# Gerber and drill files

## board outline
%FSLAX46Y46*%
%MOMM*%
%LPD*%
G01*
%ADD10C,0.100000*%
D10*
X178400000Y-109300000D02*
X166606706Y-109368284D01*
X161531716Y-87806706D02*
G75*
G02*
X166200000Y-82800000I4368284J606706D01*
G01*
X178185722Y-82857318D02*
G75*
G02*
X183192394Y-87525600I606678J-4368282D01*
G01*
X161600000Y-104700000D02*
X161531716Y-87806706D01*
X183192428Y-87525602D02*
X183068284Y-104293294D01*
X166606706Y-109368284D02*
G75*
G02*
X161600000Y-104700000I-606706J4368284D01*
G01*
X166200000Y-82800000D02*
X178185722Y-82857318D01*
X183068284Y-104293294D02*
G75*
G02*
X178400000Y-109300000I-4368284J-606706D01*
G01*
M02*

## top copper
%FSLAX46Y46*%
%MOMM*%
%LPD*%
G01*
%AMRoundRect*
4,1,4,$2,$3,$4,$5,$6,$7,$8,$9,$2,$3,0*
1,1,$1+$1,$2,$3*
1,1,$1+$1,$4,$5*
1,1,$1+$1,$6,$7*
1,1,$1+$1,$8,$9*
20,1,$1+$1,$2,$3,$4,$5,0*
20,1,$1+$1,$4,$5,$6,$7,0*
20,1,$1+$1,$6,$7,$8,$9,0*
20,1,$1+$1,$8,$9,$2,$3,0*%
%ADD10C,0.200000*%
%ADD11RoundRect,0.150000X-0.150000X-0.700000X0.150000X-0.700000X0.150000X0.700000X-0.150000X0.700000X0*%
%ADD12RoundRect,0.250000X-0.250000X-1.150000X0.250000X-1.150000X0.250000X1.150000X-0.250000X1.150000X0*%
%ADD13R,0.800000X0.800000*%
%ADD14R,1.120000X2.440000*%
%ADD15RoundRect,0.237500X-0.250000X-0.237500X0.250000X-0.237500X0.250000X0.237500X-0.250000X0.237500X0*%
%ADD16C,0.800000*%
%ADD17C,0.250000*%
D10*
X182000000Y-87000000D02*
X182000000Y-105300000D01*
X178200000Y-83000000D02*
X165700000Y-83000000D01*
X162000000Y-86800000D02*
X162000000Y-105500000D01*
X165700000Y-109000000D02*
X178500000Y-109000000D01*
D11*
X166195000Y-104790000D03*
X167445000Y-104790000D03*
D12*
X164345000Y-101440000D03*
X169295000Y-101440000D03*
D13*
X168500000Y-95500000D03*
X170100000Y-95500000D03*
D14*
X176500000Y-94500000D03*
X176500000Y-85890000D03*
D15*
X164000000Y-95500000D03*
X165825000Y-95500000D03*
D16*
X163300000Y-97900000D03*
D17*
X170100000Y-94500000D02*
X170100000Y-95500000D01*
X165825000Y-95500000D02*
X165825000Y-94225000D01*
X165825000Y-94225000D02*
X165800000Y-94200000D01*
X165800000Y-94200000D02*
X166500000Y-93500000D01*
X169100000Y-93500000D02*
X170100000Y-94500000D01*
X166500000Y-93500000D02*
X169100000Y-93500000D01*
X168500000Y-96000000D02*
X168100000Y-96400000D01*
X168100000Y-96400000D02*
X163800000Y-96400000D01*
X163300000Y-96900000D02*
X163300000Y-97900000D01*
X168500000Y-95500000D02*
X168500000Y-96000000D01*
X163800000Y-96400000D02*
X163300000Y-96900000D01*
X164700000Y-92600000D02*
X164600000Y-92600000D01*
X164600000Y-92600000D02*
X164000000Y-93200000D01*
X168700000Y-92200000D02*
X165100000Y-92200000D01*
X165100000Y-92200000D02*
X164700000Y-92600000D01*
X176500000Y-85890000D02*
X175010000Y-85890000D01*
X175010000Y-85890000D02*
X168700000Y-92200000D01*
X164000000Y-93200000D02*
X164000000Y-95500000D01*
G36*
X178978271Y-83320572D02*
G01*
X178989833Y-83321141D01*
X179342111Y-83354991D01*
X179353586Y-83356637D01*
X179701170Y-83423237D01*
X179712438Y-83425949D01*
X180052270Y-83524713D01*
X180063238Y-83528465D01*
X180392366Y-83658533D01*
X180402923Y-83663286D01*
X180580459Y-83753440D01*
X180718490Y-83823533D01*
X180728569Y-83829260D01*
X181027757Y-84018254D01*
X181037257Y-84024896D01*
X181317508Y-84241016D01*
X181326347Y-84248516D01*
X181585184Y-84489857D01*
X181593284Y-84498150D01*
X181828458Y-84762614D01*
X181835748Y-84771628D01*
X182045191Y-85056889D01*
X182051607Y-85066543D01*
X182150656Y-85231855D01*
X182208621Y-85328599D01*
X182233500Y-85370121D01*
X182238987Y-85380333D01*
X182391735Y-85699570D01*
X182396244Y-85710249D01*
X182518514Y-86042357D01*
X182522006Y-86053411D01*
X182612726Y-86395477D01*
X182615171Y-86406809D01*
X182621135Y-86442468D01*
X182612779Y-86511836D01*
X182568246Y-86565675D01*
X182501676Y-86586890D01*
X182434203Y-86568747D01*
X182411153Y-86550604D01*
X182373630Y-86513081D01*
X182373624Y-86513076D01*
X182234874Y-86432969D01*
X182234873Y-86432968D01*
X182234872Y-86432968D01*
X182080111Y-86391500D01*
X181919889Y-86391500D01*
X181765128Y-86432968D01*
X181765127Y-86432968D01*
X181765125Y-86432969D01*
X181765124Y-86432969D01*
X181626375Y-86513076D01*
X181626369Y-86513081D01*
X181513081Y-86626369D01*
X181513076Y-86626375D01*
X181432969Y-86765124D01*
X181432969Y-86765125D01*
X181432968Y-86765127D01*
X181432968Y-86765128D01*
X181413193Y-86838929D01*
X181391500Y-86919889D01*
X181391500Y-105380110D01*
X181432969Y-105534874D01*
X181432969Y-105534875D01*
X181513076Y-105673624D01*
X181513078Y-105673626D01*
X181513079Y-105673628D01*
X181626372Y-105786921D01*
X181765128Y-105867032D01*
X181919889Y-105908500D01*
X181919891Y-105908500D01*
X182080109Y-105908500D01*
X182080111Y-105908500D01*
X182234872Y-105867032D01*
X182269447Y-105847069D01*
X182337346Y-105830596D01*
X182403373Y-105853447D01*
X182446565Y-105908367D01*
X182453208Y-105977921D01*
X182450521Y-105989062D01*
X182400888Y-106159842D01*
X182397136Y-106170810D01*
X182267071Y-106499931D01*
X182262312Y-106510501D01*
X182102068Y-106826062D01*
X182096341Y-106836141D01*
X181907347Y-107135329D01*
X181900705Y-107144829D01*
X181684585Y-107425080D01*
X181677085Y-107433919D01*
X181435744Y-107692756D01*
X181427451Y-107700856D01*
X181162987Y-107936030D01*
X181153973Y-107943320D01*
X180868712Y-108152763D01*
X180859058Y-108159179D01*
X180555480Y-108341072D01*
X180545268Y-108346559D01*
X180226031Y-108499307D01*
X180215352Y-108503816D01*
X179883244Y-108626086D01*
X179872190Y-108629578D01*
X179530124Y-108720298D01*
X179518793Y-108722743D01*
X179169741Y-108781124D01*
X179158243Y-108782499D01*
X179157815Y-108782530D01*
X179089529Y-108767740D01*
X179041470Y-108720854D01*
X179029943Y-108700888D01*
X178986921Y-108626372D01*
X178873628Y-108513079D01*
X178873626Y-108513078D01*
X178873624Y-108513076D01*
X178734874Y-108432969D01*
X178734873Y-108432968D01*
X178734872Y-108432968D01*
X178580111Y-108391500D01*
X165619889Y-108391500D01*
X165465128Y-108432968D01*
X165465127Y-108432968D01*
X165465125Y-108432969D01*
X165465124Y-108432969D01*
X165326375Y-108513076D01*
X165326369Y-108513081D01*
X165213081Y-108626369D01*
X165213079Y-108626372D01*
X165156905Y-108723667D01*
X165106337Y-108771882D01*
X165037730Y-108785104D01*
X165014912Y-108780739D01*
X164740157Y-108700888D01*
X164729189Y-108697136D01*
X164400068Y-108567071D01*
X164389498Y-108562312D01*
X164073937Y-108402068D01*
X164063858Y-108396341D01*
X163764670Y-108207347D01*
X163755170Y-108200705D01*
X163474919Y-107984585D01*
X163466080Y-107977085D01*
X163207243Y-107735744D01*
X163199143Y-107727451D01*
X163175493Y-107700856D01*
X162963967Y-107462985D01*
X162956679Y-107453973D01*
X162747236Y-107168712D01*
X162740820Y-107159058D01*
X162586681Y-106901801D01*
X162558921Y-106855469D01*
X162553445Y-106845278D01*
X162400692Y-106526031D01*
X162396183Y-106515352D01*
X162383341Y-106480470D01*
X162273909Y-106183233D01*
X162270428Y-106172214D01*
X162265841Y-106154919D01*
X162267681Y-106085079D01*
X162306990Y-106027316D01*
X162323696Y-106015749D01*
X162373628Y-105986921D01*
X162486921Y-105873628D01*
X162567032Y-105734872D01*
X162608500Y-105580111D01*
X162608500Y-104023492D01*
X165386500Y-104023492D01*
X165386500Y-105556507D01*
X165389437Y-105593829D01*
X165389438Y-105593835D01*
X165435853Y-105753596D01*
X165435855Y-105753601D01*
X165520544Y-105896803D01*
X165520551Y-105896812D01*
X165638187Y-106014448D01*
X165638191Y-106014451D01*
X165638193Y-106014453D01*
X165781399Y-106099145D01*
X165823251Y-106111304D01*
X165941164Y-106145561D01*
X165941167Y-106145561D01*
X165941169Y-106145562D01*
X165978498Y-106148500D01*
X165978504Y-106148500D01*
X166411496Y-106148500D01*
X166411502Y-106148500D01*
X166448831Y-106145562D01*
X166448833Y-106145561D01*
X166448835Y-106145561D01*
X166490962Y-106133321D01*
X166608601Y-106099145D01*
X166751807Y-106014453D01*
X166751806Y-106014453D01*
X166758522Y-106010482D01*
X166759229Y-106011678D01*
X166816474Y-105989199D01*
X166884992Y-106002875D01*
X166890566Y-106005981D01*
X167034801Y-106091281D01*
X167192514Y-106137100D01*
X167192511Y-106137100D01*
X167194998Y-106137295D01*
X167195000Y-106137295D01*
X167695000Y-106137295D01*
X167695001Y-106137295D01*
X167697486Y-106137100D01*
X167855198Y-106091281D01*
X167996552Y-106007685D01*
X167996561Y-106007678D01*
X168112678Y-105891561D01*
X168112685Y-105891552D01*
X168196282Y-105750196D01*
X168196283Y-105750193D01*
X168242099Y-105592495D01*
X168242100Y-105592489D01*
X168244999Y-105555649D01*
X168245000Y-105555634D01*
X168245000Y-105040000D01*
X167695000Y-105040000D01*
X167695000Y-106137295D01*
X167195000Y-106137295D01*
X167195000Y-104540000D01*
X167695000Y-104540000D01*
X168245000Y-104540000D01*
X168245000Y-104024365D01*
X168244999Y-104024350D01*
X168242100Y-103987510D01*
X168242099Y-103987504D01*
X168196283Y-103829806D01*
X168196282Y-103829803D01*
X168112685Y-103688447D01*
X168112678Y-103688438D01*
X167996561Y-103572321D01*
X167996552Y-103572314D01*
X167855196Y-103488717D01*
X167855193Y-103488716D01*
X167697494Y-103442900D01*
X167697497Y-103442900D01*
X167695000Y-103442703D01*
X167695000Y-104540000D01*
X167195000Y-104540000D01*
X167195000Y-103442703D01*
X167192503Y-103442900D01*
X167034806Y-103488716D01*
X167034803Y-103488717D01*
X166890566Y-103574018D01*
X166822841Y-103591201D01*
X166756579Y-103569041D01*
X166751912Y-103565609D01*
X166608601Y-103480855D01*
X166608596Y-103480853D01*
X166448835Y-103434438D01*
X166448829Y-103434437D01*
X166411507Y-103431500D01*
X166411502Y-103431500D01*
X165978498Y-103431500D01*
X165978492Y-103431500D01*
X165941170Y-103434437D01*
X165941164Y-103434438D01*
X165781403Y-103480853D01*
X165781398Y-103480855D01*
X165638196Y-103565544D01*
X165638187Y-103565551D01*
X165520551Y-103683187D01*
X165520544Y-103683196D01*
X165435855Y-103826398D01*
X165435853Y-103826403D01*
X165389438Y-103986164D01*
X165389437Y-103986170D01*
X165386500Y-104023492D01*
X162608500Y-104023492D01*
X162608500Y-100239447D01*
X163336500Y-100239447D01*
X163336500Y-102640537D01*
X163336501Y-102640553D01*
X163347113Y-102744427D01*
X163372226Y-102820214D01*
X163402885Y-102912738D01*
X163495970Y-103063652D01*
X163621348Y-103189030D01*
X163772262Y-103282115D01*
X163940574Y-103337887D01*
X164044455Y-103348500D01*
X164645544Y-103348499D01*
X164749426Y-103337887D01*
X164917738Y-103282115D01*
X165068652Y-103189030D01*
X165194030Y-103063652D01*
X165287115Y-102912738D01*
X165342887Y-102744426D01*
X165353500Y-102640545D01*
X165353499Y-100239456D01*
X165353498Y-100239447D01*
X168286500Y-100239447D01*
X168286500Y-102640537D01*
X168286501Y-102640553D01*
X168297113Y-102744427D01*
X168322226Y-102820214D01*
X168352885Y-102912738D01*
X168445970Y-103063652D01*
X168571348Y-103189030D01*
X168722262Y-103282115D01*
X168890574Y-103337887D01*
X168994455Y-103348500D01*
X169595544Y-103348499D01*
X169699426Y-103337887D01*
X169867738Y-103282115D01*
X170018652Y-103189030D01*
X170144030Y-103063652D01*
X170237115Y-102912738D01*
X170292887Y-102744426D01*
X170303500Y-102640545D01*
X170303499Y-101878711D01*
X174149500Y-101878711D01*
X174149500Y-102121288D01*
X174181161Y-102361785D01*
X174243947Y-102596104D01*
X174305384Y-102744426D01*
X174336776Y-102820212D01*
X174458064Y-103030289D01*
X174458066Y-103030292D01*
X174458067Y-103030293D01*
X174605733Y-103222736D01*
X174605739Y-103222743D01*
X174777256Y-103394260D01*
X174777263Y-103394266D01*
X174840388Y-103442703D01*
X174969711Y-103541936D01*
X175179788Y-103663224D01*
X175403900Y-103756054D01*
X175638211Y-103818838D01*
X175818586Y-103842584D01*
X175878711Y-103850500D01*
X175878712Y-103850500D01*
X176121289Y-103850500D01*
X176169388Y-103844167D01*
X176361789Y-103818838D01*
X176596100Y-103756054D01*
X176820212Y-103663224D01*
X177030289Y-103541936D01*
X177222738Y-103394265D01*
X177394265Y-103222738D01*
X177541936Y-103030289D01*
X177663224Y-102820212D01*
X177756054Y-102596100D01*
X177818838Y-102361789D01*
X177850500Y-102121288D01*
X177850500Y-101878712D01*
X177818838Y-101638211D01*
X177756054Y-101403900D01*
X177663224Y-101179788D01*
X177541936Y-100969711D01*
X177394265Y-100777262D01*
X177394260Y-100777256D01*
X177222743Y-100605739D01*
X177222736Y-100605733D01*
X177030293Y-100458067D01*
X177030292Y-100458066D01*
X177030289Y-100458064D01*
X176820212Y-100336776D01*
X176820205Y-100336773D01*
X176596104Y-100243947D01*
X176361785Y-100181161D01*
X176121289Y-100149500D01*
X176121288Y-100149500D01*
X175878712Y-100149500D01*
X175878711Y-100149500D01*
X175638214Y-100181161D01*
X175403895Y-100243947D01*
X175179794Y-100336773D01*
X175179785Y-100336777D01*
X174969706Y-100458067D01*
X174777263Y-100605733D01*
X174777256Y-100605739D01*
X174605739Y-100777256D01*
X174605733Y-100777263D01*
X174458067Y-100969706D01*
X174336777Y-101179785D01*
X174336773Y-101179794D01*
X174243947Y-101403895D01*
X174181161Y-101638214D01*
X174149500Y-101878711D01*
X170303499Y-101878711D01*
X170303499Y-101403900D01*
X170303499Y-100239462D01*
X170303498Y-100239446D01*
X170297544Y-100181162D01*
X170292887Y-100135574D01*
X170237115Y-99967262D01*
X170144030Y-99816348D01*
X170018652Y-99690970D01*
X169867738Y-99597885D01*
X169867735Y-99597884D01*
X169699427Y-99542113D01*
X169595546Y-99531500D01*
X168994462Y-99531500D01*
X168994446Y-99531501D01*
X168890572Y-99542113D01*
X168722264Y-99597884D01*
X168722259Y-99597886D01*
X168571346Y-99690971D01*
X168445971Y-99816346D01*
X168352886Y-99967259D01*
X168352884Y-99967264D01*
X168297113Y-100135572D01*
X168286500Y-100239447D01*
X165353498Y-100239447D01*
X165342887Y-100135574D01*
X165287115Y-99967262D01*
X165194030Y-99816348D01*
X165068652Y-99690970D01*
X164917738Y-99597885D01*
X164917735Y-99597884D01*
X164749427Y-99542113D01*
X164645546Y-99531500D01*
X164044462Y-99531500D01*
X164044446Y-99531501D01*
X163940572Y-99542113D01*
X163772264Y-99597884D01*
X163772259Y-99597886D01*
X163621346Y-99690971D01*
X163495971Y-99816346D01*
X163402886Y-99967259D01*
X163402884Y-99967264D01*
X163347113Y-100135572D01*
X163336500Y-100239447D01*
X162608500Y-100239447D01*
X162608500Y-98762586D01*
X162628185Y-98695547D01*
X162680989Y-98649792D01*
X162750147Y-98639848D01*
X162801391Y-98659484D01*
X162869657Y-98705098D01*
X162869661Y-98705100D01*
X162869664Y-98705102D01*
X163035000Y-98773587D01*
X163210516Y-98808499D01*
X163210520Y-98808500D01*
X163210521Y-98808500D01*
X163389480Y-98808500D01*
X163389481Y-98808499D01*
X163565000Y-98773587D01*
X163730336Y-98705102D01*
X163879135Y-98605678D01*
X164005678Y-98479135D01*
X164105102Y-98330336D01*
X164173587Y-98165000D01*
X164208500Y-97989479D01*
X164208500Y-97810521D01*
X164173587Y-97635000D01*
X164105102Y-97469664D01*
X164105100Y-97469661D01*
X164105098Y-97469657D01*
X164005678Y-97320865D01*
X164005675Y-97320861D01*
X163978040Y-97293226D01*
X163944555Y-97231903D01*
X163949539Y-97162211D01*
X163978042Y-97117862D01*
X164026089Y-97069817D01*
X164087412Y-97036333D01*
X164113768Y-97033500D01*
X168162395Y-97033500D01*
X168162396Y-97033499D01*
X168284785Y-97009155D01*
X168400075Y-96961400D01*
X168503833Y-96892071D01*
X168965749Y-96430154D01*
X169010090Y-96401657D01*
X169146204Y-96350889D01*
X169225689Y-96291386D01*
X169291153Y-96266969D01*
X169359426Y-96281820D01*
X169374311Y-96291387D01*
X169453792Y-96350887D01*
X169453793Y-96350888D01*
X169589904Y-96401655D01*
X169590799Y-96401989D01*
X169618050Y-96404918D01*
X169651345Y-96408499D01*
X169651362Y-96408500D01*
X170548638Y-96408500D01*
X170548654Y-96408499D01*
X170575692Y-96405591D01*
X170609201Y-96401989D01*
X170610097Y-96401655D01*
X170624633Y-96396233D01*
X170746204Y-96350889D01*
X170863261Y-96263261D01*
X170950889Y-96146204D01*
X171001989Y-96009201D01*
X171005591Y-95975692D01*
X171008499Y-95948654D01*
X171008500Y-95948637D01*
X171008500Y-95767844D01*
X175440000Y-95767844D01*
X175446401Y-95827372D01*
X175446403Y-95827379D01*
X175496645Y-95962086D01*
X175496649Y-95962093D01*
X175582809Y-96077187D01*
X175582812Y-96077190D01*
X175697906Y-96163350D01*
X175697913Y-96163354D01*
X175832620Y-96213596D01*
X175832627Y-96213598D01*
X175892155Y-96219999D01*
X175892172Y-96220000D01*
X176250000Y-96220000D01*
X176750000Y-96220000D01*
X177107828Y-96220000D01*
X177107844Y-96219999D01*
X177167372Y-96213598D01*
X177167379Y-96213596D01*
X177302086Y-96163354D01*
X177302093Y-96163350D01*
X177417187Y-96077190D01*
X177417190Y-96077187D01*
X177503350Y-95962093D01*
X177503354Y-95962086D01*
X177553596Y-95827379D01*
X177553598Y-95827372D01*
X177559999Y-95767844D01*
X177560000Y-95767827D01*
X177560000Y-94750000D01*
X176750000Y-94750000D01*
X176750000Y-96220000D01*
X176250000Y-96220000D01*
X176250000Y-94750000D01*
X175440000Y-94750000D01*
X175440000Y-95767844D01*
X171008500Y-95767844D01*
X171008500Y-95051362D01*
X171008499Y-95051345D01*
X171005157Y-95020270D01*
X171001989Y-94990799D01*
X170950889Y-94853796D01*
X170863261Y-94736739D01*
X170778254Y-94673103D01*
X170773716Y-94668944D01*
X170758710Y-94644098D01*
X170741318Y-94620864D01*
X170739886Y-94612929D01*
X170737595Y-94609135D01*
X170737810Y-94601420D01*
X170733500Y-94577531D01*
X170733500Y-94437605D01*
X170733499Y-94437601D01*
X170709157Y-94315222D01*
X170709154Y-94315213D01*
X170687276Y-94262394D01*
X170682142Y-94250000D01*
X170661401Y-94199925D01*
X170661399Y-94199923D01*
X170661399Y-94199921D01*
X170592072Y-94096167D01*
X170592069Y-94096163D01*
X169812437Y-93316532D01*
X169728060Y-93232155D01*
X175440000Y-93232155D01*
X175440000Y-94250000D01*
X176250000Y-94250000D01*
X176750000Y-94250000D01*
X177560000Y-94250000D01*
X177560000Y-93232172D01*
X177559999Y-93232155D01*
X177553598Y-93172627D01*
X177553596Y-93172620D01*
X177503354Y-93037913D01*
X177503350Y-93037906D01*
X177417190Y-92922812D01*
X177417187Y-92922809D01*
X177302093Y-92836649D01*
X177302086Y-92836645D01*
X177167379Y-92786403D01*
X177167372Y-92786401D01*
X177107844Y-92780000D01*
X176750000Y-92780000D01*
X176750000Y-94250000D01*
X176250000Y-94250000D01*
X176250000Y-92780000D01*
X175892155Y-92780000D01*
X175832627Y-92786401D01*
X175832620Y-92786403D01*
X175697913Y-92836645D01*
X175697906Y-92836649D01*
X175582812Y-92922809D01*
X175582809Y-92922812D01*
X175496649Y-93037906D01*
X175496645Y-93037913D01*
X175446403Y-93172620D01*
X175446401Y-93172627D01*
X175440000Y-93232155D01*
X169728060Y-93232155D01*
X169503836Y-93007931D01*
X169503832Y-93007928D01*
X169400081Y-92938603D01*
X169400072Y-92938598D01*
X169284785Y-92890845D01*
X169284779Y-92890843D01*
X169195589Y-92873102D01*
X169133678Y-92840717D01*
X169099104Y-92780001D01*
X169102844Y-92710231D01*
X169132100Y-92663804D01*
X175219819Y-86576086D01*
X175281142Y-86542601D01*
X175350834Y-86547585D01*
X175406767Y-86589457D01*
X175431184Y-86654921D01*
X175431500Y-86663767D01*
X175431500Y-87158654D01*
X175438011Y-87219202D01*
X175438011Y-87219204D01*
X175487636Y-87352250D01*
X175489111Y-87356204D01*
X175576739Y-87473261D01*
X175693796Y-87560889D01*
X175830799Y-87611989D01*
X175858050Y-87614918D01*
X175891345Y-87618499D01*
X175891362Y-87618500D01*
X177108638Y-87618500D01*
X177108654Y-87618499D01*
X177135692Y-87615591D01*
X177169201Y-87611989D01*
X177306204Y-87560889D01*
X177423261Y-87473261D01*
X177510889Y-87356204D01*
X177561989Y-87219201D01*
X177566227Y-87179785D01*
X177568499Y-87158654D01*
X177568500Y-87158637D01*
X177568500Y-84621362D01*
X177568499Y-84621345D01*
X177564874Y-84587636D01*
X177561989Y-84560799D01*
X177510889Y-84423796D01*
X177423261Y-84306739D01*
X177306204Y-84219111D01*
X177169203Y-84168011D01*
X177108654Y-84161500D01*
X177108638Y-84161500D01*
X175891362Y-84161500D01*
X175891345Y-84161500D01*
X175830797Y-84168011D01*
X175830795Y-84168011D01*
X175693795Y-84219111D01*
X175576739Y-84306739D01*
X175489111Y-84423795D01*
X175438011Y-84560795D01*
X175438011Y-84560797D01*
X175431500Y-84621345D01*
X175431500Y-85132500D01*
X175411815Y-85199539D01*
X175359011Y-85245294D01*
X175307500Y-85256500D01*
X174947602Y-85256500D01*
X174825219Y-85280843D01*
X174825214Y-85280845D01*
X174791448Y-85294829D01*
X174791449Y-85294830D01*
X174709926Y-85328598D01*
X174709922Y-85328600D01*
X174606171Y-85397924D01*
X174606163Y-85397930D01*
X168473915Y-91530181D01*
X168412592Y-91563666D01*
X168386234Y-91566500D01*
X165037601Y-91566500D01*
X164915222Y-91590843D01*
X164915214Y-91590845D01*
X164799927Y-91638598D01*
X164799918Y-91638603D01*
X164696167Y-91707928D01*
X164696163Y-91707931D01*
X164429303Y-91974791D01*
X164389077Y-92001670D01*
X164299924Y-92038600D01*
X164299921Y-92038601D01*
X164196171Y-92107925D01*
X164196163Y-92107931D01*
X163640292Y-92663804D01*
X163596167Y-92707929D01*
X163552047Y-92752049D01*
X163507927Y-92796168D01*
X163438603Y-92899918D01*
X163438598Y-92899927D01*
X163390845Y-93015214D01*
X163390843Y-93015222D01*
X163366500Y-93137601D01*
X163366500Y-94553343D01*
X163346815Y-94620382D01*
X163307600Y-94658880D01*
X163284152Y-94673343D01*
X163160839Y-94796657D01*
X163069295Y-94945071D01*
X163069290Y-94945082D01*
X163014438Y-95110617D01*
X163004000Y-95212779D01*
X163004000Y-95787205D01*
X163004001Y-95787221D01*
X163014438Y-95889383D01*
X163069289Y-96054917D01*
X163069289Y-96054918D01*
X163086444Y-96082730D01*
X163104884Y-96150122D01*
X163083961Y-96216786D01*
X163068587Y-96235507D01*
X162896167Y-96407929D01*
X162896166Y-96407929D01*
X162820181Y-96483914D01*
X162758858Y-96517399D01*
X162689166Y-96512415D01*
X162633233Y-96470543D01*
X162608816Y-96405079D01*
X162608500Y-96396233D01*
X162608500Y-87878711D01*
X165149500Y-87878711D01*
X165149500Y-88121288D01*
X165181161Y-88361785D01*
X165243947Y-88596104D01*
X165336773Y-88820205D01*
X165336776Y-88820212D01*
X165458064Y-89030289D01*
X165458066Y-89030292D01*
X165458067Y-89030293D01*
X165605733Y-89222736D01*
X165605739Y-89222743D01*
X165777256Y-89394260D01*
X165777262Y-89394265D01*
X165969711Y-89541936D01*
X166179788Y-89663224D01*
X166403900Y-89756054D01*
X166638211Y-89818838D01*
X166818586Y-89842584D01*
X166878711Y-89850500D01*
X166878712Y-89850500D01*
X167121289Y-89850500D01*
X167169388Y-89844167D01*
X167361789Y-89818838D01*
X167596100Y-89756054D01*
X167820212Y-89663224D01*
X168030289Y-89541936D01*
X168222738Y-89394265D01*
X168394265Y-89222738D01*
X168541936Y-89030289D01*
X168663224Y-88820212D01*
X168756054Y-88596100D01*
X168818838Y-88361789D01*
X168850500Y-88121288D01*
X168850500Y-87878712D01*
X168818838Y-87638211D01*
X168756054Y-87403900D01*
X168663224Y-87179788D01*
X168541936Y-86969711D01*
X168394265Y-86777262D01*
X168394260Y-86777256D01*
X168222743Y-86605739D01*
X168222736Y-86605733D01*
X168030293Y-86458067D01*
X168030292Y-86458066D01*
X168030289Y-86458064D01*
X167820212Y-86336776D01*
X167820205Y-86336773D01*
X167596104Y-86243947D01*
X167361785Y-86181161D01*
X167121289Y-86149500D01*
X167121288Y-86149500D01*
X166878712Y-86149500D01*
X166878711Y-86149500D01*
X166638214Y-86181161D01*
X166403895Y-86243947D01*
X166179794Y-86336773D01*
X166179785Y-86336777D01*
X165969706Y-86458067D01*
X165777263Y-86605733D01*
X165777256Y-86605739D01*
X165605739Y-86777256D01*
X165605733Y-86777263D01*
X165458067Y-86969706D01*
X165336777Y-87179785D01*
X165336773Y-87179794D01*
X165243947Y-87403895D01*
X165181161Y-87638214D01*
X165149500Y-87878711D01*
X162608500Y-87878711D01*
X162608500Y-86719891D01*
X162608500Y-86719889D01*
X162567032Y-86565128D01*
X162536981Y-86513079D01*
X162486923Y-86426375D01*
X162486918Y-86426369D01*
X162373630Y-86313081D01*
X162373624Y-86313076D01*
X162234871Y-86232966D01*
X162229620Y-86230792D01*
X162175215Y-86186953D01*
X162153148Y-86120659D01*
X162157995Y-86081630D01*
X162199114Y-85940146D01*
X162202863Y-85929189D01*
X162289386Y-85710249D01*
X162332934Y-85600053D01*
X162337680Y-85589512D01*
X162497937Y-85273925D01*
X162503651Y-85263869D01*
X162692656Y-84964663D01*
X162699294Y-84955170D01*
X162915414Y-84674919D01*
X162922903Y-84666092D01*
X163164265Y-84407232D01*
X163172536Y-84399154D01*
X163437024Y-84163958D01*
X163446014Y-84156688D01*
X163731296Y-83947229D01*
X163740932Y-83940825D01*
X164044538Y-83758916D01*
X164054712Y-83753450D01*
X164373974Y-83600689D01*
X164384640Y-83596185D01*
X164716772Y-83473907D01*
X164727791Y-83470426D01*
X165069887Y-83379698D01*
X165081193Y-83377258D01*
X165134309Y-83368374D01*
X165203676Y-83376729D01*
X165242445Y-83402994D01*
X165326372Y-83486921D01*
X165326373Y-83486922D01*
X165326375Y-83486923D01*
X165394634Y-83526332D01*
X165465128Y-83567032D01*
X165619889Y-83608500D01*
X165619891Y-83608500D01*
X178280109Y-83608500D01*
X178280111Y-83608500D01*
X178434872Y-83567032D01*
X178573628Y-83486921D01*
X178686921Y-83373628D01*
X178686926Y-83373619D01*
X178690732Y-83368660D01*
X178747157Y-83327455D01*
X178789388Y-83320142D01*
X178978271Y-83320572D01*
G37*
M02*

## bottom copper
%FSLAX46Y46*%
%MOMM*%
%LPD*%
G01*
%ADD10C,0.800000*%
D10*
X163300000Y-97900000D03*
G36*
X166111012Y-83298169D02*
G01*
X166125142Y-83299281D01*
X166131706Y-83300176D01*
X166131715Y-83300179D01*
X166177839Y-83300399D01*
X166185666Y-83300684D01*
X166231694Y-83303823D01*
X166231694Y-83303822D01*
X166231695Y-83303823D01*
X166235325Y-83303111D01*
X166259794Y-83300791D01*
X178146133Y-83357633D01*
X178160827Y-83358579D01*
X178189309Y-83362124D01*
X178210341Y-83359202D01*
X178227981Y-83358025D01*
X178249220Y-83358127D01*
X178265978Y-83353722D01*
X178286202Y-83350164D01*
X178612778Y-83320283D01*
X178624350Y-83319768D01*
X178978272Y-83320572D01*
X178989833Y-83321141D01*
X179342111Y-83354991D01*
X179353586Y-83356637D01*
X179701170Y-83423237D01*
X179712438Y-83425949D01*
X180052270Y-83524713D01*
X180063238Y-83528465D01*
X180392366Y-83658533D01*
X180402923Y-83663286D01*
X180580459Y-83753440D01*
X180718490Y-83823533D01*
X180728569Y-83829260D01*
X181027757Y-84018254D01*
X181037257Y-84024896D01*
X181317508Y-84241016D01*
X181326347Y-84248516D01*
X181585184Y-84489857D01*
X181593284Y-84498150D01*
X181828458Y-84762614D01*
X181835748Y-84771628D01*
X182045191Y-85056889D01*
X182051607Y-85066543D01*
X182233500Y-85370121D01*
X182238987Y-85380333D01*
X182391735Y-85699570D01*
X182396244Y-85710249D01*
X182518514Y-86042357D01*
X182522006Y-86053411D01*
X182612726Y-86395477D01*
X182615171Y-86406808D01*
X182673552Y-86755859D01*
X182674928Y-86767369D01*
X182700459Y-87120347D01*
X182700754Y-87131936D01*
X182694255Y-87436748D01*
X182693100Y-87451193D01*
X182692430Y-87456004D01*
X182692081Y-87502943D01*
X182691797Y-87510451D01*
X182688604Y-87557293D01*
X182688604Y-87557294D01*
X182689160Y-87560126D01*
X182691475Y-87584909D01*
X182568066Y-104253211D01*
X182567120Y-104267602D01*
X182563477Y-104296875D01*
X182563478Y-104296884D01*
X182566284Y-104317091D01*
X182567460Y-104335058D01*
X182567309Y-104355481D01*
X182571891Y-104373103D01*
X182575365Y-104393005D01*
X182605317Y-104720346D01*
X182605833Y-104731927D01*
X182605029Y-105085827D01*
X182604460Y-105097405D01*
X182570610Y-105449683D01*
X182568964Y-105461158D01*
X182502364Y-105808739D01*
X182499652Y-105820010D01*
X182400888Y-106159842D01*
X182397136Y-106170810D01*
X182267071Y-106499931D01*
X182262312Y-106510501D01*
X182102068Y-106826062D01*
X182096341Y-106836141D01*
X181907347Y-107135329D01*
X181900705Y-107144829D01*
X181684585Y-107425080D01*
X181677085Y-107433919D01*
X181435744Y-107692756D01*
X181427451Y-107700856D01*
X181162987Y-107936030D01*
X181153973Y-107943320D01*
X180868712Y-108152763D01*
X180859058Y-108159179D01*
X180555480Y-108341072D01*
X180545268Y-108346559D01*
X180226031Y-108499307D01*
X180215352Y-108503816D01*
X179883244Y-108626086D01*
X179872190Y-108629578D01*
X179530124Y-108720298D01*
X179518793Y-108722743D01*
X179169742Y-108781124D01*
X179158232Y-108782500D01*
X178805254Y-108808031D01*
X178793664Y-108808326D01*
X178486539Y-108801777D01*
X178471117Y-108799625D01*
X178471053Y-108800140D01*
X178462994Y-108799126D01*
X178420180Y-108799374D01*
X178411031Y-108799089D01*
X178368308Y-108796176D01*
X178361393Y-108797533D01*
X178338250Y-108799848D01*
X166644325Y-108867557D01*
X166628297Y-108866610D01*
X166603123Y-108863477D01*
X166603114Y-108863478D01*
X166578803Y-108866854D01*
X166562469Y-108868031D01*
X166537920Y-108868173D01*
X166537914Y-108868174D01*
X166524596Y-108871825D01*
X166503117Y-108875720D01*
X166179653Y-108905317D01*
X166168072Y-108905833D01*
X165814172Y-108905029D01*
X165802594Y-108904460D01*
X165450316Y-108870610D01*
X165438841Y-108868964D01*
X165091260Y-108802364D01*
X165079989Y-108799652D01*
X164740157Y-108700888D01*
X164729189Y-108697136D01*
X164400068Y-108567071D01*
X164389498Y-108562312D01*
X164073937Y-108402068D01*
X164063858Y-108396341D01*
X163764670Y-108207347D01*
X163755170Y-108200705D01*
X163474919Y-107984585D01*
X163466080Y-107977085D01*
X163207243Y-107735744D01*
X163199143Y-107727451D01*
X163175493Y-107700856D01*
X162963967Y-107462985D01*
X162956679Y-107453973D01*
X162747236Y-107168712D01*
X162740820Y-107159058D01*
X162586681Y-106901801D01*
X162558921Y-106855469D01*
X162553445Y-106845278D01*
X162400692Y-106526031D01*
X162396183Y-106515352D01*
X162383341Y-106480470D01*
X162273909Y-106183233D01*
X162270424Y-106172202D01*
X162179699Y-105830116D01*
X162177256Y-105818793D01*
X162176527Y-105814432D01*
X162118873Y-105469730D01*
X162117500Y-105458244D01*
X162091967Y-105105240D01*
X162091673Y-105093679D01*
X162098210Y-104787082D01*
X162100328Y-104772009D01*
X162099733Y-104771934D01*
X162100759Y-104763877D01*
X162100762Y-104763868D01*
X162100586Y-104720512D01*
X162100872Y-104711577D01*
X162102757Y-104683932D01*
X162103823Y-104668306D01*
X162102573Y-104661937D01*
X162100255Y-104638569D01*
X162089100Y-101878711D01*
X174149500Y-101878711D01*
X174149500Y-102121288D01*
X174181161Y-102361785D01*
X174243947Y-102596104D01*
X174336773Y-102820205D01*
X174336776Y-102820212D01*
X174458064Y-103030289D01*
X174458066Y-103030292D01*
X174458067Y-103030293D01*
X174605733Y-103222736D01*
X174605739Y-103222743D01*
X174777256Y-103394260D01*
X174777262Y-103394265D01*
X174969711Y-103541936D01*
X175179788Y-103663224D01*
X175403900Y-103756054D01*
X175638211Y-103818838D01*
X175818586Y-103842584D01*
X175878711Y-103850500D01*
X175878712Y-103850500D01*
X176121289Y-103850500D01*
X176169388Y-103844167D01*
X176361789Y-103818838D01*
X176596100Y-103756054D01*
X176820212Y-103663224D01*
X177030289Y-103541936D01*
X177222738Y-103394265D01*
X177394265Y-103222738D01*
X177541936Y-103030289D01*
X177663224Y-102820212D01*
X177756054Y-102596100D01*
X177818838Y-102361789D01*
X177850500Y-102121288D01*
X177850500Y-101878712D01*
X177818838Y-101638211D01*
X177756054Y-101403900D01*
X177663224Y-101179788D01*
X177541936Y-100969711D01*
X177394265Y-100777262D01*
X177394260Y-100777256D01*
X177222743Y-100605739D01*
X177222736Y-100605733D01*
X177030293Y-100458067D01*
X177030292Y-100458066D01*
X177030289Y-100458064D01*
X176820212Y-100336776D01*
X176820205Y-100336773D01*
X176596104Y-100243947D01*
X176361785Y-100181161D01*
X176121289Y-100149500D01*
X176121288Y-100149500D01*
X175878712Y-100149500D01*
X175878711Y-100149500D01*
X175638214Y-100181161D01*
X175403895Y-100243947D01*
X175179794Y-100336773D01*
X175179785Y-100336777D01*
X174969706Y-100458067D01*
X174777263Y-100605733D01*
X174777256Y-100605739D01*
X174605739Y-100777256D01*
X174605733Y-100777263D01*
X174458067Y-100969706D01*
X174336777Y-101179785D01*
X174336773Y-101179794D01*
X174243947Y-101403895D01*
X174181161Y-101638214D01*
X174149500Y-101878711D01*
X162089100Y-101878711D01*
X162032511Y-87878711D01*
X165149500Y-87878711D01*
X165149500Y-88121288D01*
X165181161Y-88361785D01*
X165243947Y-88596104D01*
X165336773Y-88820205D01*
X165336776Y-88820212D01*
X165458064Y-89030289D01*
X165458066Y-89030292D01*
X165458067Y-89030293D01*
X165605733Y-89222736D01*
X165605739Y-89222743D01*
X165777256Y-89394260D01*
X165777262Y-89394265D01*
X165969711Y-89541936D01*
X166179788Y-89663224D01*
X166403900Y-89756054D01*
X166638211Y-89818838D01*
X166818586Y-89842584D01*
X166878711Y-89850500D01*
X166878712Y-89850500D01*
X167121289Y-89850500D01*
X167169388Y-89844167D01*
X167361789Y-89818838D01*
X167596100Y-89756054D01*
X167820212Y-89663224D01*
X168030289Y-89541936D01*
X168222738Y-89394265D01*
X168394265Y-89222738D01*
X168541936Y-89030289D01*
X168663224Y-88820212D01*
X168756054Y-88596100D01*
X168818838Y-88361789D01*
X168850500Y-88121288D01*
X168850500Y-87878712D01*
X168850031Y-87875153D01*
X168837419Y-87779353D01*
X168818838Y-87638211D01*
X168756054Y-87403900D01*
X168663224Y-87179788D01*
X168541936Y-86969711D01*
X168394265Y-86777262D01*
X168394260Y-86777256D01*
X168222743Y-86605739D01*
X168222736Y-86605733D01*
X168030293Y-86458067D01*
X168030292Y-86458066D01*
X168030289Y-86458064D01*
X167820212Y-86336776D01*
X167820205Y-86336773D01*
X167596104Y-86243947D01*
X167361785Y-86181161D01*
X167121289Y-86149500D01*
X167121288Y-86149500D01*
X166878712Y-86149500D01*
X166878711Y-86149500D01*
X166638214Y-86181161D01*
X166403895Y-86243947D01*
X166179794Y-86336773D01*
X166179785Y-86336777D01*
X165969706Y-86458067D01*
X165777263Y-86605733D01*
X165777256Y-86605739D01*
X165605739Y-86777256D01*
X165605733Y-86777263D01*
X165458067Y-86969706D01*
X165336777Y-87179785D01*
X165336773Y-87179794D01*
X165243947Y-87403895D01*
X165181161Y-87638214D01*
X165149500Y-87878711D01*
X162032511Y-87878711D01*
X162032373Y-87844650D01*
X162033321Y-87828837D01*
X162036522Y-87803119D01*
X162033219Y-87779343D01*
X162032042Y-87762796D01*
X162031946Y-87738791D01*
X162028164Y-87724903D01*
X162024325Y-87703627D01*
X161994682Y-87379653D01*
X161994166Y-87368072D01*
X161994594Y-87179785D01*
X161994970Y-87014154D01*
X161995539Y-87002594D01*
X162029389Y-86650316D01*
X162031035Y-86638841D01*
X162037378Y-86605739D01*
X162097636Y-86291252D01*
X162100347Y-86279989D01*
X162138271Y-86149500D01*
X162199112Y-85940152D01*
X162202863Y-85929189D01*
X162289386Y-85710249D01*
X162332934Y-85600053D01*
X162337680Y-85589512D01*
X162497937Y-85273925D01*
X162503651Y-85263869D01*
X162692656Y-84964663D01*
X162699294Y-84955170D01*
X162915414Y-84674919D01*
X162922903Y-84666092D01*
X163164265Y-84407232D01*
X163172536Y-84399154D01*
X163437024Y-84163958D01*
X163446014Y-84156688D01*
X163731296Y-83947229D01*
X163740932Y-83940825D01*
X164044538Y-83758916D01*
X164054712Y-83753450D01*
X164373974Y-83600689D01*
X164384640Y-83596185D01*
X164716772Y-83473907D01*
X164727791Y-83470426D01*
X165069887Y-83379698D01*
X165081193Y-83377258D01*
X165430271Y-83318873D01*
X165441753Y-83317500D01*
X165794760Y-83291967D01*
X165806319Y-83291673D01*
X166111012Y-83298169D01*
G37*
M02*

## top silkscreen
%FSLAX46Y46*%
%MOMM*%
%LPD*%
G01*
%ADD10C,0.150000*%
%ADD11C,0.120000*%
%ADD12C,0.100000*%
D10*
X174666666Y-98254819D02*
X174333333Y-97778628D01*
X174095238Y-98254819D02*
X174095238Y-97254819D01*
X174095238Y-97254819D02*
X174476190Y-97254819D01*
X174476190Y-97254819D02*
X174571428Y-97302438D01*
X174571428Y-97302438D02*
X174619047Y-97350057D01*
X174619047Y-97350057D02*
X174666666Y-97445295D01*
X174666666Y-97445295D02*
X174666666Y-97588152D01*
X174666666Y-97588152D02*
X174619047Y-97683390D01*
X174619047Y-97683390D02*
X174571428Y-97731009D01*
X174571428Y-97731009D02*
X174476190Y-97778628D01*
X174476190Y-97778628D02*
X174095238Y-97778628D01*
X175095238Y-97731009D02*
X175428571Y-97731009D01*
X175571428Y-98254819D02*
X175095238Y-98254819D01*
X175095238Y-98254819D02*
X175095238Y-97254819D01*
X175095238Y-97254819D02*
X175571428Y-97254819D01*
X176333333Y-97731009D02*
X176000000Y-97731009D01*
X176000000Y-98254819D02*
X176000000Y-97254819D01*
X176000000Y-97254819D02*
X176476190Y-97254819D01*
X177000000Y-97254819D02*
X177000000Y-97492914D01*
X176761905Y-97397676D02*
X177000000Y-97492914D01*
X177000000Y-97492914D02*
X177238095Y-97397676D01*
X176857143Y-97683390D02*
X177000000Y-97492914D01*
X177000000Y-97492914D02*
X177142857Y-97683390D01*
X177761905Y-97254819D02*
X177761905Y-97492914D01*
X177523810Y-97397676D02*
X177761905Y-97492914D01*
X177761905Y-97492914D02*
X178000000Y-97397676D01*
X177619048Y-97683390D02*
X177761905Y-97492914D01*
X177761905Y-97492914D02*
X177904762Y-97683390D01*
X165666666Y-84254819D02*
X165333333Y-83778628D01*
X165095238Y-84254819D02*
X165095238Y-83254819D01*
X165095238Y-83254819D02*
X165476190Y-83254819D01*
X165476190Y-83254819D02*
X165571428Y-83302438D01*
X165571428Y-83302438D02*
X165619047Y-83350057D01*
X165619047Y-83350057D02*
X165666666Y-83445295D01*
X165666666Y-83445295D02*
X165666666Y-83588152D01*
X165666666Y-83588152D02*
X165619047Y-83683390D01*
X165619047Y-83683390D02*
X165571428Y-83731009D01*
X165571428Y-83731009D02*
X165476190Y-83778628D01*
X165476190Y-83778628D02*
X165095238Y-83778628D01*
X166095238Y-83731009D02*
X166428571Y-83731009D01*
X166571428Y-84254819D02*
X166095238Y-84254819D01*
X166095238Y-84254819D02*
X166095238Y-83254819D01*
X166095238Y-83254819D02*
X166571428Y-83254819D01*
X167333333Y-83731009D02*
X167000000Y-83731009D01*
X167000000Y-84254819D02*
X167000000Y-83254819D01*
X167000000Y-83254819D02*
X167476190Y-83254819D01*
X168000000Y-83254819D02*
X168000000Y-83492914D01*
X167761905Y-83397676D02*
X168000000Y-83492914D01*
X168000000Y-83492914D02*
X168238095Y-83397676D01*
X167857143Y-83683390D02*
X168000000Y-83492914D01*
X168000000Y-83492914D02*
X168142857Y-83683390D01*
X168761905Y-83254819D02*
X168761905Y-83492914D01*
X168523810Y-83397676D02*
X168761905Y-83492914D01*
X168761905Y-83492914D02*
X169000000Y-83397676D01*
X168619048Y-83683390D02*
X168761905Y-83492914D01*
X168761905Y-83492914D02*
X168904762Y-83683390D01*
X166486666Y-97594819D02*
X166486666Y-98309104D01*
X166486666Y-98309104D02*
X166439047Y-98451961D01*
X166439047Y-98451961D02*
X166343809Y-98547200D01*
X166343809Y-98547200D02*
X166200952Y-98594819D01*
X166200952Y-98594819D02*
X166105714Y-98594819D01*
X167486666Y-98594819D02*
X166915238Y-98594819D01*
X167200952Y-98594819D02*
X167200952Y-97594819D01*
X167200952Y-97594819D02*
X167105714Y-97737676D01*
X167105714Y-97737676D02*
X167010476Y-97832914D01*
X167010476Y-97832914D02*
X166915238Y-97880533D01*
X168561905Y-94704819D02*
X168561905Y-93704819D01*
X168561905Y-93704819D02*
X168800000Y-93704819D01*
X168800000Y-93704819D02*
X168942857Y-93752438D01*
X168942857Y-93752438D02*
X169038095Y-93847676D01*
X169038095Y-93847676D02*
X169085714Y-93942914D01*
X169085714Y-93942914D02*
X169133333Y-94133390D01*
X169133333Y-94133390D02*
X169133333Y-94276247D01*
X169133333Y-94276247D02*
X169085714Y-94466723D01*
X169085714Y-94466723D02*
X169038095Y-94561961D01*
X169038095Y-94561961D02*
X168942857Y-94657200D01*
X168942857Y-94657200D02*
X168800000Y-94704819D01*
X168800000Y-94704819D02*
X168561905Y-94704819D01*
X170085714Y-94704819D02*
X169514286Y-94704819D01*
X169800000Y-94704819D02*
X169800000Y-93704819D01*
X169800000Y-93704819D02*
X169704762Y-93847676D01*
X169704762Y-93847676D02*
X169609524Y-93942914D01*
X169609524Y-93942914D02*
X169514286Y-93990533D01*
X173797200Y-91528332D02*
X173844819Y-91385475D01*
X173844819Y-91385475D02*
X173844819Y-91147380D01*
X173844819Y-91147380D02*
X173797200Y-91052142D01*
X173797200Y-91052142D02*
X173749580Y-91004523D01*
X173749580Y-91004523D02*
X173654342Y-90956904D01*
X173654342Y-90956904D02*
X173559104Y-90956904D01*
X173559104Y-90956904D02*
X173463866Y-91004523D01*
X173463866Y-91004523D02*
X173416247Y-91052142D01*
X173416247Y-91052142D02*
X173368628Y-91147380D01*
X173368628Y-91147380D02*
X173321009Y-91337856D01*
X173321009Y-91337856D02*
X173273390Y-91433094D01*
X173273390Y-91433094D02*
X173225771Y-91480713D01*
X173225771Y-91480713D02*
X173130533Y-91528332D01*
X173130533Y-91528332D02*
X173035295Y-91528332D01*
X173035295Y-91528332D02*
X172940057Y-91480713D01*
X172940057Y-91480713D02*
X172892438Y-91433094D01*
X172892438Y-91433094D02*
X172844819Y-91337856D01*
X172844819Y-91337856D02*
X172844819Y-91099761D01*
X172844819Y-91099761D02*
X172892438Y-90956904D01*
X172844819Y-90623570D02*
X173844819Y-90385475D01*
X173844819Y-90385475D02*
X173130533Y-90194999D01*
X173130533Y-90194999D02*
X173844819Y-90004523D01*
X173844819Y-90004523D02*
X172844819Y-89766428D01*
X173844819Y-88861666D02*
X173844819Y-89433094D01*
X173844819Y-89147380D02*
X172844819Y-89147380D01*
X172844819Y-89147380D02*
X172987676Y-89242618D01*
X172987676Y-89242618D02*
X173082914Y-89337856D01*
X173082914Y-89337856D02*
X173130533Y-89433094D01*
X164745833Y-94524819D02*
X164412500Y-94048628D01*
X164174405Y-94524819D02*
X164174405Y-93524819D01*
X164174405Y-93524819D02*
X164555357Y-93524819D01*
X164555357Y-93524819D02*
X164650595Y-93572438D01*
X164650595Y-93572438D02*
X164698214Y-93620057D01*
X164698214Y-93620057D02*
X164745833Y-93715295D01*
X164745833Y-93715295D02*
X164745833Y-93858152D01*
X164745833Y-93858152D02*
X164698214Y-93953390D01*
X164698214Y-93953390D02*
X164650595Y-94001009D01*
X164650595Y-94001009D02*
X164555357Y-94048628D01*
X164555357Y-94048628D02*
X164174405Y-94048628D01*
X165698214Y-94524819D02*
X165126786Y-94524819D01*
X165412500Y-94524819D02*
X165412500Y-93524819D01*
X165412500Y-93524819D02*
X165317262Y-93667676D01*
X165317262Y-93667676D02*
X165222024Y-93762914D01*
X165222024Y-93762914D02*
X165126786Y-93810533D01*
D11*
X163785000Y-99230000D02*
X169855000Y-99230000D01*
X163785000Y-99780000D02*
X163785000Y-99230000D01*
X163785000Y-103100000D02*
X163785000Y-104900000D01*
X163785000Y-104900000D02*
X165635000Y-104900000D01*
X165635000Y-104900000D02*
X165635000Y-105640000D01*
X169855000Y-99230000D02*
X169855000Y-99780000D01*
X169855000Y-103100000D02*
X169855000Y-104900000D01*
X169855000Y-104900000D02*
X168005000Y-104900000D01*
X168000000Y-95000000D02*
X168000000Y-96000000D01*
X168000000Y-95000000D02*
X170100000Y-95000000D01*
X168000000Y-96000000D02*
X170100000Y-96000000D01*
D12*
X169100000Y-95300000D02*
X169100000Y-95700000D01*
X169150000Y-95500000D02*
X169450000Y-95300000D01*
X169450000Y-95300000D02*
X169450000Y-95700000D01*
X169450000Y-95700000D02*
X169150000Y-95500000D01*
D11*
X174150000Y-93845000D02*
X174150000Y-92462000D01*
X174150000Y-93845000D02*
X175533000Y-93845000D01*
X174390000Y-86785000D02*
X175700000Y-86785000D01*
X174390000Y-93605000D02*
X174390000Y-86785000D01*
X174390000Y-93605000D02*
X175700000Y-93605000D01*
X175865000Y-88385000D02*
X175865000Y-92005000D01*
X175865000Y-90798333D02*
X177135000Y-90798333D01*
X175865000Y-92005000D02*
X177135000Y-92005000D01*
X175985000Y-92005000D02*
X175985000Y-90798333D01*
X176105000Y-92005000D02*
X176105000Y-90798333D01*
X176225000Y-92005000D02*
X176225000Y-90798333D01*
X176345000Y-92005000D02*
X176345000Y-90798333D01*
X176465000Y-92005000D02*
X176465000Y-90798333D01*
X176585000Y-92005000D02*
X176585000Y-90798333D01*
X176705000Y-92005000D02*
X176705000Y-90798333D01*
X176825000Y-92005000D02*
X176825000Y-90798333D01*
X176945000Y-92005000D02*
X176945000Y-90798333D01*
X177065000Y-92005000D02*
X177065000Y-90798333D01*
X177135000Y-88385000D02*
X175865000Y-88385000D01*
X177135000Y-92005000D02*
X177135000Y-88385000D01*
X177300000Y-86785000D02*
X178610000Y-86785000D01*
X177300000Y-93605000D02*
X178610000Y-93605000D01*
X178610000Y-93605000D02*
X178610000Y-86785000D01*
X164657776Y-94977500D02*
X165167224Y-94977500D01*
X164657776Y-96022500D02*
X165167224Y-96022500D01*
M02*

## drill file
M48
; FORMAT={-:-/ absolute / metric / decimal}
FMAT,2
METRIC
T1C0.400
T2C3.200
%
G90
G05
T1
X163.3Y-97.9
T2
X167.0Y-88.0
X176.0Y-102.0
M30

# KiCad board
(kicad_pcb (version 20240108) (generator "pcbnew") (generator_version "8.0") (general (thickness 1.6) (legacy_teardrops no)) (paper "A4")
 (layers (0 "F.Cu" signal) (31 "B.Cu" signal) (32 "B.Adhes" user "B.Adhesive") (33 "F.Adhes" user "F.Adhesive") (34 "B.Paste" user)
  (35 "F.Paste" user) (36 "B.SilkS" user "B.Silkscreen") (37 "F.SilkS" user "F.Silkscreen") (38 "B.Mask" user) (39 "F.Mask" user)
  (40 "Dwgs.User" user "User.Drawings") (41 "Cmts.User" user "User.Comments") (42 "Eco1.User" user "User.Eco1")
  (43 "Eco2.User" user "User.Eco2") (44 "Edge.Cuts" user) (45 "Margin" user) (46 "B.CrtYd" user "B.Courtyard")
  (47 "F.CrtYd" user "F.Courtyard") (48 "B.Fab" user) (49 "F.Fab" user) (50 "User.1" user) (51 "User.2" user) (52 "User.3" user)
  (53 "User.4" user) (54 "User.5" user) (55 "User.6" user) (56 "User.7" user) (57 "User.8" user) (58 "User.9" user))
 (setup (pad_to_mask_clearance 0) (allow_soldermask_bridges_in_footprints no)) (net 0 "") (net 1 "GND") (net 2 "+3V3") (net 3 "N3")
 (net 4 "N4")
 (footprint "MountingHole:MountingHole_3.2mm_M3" (layer "F.Cu") (at 176 102)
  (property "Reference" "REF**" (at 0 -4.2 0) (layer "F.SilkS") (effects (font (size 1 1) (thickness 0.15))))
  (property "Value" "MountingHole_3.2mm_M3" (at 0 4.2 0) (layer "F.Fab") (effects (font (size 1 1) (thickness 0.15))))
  (pad "" np_thru_hole circle (at 0 0) (size 3.2 3.2) (drill 3.2) (layers "*.Cu" "*.Mask")))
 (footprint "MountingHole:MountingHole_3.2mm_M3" (layer "F.Cu") (at 167 88)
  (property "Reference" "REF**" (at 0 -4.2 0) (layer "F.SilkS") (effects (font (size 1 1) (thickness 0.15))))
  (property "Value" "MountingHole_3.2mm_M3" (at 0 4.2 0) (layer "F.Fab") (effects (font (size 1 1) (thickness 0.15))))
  (pad "" np_thru_hole circle (at 0 0) (size 3.2 3.2) (drill 3.2) (layers "*.Cu" "*.Mask")))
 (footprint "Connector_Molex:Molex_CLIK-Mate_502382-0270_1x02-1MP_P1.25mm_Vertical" (layer "F.Cu") (at 166.82 102.84)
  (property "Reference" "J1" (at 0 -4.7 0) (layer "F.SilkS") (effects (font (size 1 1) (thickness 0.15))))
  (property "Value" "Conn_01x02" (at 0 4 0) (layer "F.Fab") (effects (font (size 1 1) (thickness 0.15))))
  (fp_line (start -3.035 -3.61) (end 3.035 -3.61) (stroke (width 0.12) (type solid)) (layer "F.SilkS"))
  (fp_line (start -3.035 -3.06) (end -3.035 -3.61) (stroke (width 0.12) (type solid)) (layer "F.SilkS"))
  (fp_line (start -3.035 0.26) (end -3.035 2.06) (stroke (width 0.12) (type solid)) (layer "F.SilkS"))
  (fp_line (start -3.035 2.06) (end -1.185 2.06) (stroke (width 0.12) (type solid)) (layer "F.SilkS"))
  (fp_line (start -1.185 2.06) (end -1.185 2.8) (stroke (width 0.12) (type solid)) (layer "F.SilkS"))
  (fp_line (start 3.035 -3.61) (end 3.035 -3.06) (stroke (width 0.12) (type solid)) (layer "F.SilkS"))
  (fp_line (start 3.035 0.26) (end 3.035 2.06) (stroke (width 0.12) (type solid)) (layer "F.SilkS"))
  (fp_line (start 3.035 2.06) (end 1.185 2.06) (stroke (width 0.12) (type solid)) (layer "F.SilkS"))
  (pad "1" smd roundrect (at -0.625 1.95) (size 0.6 1.7) (layers "F.Cu" "F.Paste" "F.Mask") (roundrect_rratio 0.25) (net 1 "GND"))
  (pad "2" smd roundrect (at 0.625 1.95) (size 0.6 1.7) (layers "F.Cu" "F.Paste" "F.Mask") (roundrect_rratio 0.25) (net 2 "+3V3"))
  (pad "MP" smd roundrect (at -2.475 -1.4) (size 1 2.8) (layers "F.Cu" "F.Paste" "F.Mask") (roundrect_rratio 0.25))
  (pad "MP" smd roundrect (at 2.475 -1.4) (size 1 2.8) (layers "F.Cu" "F.Paste" "F.Mask") (roundrect_rratio 0.25)))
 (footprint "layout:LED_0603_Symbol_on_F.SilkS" (layer "F.Cu") (at 169.3 95.5)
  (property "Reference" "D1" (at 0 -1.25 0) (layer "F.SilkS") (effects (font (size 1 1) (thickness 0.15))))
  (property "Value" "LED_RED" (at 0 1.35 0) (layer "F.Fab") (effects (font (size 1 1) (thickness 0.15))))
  (fp_line (start -1.3 -0.5) (end -1.3 0.5) (stroke (width 0.12) (type solid)) (layer "F.SilkS"))
  (fp_line (start -1.3 -0.5) (end 0.8 -0.5) (stroke (width 0.12) (type solid)) (layer "F.SilkS"))
  (fp_line (start -1.3 0.5) (end 0.8 0.5) (stroke (width 0.12) (type solid)) (layer "F.SilkS"))
  (fp_line (start -0.2 -0.2) (end -0.2 0.2) (stroke (width 0.1) (type solid)) (layer "F.SilkS"))
  (fp_line (start -0.15 0) (end 0.15 -0.2) (stroke (width 0.1) (type solid)) (layer "F.SilkS"))
  (fp_line (start 0.15 -0.2) (end 0.15 0.2) (stroke (width 0.1) (type solid)) (layer "F.SilkS"))
  (fp_line (start 0.15 0.2) (end -0.15 0) (stroke (width 0.1) (type solid)) (layer "F.SilkS"))
  (pad "1" smd rect (at -0.8 0 180) (size 0.8 0.8) (layers "F.Cu" "F.Paste" "F.Mask") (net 1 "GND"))
  (pad "2" smd rect (at 0.8 0 180) (size 0.8 0.8) (layers "F.Cu" "F.Paste" "F.Mask") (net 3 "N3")))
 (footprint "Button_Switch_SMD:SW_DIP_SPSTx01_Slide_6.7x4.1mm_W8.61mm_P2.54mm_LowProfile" (layer "F.Cu") (at 176.5 90.195 90)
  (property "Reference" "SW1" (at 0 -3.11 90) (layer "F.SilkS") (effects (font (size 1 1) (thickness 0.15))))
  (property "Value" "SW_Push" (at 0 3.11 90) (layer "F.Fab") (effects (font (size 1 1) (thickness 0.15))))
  (fp_line (start -3.65 -2.35) (end -2.267 -2.35) (stroke (width 0.12) (type solid)) (layer "F.SilkS"))
  (fp_line (start -3.65 -2.35) (end -3.65 -0.967) (stroke (width 0.12) (type solid)) (layer "F.SilkS"))
  (fp_line (start 3.41 -2.11) (end 3.41 -0.8) (stroke (width 0.12) (type solid)) (layer "F.SilkS"))
  (fp_line (start -3.41 -2.11) (end 3.41 -2.11) (stroke (width 0.12) (type solid)) (layer "F.SilkS"))
  (fp_line (start -3.41 -2.11) (end -3.41 -0.8) (stroke (width 0.12) (type solid)) (layer "F.SilkS"))
  (fp_line (start 1.81 -0.635) (end -1.81 -0.635) (stroke (width 0.12) (type solid)) (layer "F.SilkS"))
  (fp_line (start -0.603333 -0.635) (end -0.603333 0.635) (stroke (width 0.12) (type solid)) (layer "F.SilkS"))
  (fp_line (start -1.81 -0.635) (end -1.81 0.635) (stroke (width 0.12) (type solid)) (layer "F.SilkS"))
  (fp_line (start -1.81 -0.515) (end -0.603333 -0.515) (stroke (width 0.12) (type solid)) (layer "F.SilkS"))
  (fp_line (start -1.81 -0.395) (end -0.603333 -0.395) (stroke (width 0.12) (type solid)) (layer "F.SilkS"))
  (fp_line (start -1.81 -0.275) (end -0.603333 -0.275) (stroke (width 0.12) (type solid)) (layer "F.SilkS"))
  (fp_line (start -1.81 -0.155) (end -0.603333 -0.155) (stroke (width 0.12) (type solid)) (layer "F.SilkS"))
  (fp_line (start -1.81 -0.035) (end -0.603333 -0.035) (stroke (width 0.12) (type solid)) (layer "F.SilkS"))
  (fp_line (start -1.81 0.085) (end -0.603333 0.085) (stroke (width 0.12) (type solid)) (layer "F.SilkS"))
  (fp_line (start -1.81 0.205) (end -0.603333 0.205) (stroke (width 0.12) (type solid)) (layer "F.SilkS"))
  (fp_line (start -1.81 0.325) (end -0.603333 0.325) (stroke (width 0.12) (type solid)) (layer "F.SilkS"))
  (fp_line (start -1.81 0.445) (end -0.603333 0.445) (stroke (width 0.12) (type solid)) (layer "F.SilkS"))
  (fp_line (start -1.81 0.565) (end -0.603333 0.565) (stroke (width 0.12) (type solid)) (layer "F.SilkS"))
  (fp_line (start 1.81 0.635) (end 1.81 -0.635) (stroke (width 0.12) (type solid)) (layer "F.SilkS"))
  (fp_line (start -1.81 0.635) (end 1.81 0.635) (stroke (width 0.12) (type solid)) (layer "F.SilkS"))
  (fp_line (start 3.41 0.8) (end 3.41 2.11) (stroke (width 0.12) (type solid)) (layer "F.SilkS"))
  (fp_line (start -3.41 0.8) (end -3.41 2.11) (stroke (width 0.12) (type solid)) (layer "F.SilkS"))
  (fp_line (start -3.41 2.11) (end 3.41 2.11) (stroke (width 0.12) (type solid)) (layer "F.SilkS"))
  (pad "1" smd rect (at -4.305 0 90) (size 2.44 1.12) (layers "F.Cu" "F.Paste" "F.Mask") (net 2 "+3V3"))
  (pad "2" smd rect (at 4.305 0 90) (size 2.44 1.12) (layers "F.Cu" "F.Paste" "F.Mask") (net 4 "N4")))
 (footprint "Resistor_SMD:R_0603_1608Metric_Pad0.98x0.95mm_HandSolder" (layer "F.Cu") (at 164.9125 95.5)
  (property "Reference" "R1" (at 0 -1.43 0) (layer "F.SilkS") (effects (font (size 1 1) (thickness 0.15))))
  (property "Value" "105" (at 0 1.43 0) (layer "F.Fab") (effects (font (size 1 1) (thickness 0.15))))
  (fp_line (start -0.254724 -0.5225) (end 0.254724 -0.5225) (stroke (width 0.12) (type solid)) (layer "F.SilkS"))
  (fp_line (start -0.254724 0.5225) (end 0.254724 0.5225) (stroke (width 0.12) (type solid)) (layer "F.SilkS"))
  (pad "1" smd roundrect (at -0.9125 0) (size 0.975 0.95) (layers "F.Cu" "F.Paste" "F.Mask") (roundrect_rratio 0.25) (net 4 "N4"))
  (pad "2" smd roundrect (at 0.9125 0) (size 0.975 0.95) (layers "F.Cu" "F.Paste" "F.Mask") (roundrect_rratio 0.25) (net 3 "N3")))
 (gr_line (start 182 87) (end 182 105.3) (stroke (width 0.2) (type default)) (layer "F.Cu"))
 (gr_line (start 178.2 83) (end 165.7 83) (stroke (width 0.2) (type default)) (layer "F.Cu"))
 (gr_line (start 162 86.8) (end 162 105.5) (stroke (width 0.2) (type default)) (layer "F.Cu"))
 (gr_line (start 165.7 109) (end 178.5 109) (stroke (width 0.2) (type default)) (layer "F.Cu"))
 (gr_line (start 178.4 109.3) (end 166.606706 109.368284) (stroke (width 0.1) (type default)) (layer "Edge.Cuts"))
 (gr_arc (start 161.531716 87.806706) (mid 162.674398 84.192428) (end 166.2 82.8) (stroke (width 0.1) (type default)) (layer "Edge.Cuts"))
 (gr_arc (start 178.185722 82.857318) (mid 181.8 84) (end 183.192428 87.525602) (stroke (width 0.1) (type default)) (layer "Edge.Cuts"))
 (gr_line (start 161.6 104.7) (end 161.531716 87.806706) (stroke (width 0.1) (type default)) (layer "Edge.Cuts"))
 (gr_line (start 183.192428 87.525602) (end 183.068284 104.293294) (stroke (width 0.1) (type default)) (layer "Edge.Cuts"))
 (gr_arc (start 166.606706 109.368284) (mid 162.992428 108.225602) (end 161.6 104.7) (stroke (width 0.1) (type default)) (layer "Edge.Cuts"))
 (gr_line (start 166.2 82.8) (end 178.185722 82.857318) (stroke (width 0.1) (type default)) (layer "Edge.Cuts"))
 (gr_arc (start 183.068284 104.293294) (mid 181.925602 107.907572) (end 178.4 109.3) (stroke (width 0.1) (type default)) (layer "Edge.Cuts"))
 (segment (start 170.1 94.5) (end 170.1 95.5) (width 0.25) (layer "F.Cu") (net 3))
 (segment (start 165.825 95.5) (end 165.825 94.225) (width 0.25) (layer "F.Cu") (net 3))
 (segment (start 165.825 94.225) (end 165.8 94.2) (width 0.25) (layer "F.Cu") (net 3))
 (segment (start 165.8 94.2) (end 166.5 93.5) (width 0.25) (layer "F.Cu") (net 3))
 (segment (start 169.1 93.5) (end 170.1 94.5) (width 0.25) (layer "F.Cu") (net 3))
 (segment (start 166.5 93.5) (end 169.1 93.5) (width 0.25) (layer "F.Cu") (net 3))
 (segment (start 168.5 96) (end 168.1 96.4) (width 0.25) (layer "F.Cu") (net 1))
 (segment (start 168.1 96.4) (end 163.8 96.4) (width 0.25) (layer "F.Cu") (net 1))
 (segment (start 163.3 96.9) (end 163.3 97.9) (width 0.25) (layer "F.Cu") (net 1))
 (segment (start 168.5 95.5) (end 168.5 96) (width 0.25) (layer "F.Cu") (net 1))
 (segment (start 163.8 96.4) (end 163.3 96.9) (width 0.25) (layer "F.Cu") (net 1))
 (via (at 163.3 97.9) (size 0.8) (drill 0.4) (layers "F.Cu" "B.Cu") (free yes) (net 1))
 (segment (start 164.7 92.6) (end 164.6 92.6) (width 0.25) (layer "F.Cu") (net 4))
 (segment (start 164.6 92.6) (end 164 93.2) (width 0.25) (layer "F.Cu") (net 4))
 (segment (start 168.7 92.2) (end 165.1 92.2) (width 0.25) (layer "F.Cu") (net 4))
 (segment (start 165.1 92.2) (end 164.7 92.6) (width 0.25) (layer "F.Cu") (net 4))
 (segment (start 176.5 85.89) (end 175.01 85.89) (width 0.25) (layer "F.Cu") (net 4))
 (segment (start 175.01 85.89) (end 168.7 92.2) (width 0.25) (layer "F.Cu") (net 4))
 (segment (start 164 93.2) (end 164 95.5) (width 0.25) (layer "F.Cu") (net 4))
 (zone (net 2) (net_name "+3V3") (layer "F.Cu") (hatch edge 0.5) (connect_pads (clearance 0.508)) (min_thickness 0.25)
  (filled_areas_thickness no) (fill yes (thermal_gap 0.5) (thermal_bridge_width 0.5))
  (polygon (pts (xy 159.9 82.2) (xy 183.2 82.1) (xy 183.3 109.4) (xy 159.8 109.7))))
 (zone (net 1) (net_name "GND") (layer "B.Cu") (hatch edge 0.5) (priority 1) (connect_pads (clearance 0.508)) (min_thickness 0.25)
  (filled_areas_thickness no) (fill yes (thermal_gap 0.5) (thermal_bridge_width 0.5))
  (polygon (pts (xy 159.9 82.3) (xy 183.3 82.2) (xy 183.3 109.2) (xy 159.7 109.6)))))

